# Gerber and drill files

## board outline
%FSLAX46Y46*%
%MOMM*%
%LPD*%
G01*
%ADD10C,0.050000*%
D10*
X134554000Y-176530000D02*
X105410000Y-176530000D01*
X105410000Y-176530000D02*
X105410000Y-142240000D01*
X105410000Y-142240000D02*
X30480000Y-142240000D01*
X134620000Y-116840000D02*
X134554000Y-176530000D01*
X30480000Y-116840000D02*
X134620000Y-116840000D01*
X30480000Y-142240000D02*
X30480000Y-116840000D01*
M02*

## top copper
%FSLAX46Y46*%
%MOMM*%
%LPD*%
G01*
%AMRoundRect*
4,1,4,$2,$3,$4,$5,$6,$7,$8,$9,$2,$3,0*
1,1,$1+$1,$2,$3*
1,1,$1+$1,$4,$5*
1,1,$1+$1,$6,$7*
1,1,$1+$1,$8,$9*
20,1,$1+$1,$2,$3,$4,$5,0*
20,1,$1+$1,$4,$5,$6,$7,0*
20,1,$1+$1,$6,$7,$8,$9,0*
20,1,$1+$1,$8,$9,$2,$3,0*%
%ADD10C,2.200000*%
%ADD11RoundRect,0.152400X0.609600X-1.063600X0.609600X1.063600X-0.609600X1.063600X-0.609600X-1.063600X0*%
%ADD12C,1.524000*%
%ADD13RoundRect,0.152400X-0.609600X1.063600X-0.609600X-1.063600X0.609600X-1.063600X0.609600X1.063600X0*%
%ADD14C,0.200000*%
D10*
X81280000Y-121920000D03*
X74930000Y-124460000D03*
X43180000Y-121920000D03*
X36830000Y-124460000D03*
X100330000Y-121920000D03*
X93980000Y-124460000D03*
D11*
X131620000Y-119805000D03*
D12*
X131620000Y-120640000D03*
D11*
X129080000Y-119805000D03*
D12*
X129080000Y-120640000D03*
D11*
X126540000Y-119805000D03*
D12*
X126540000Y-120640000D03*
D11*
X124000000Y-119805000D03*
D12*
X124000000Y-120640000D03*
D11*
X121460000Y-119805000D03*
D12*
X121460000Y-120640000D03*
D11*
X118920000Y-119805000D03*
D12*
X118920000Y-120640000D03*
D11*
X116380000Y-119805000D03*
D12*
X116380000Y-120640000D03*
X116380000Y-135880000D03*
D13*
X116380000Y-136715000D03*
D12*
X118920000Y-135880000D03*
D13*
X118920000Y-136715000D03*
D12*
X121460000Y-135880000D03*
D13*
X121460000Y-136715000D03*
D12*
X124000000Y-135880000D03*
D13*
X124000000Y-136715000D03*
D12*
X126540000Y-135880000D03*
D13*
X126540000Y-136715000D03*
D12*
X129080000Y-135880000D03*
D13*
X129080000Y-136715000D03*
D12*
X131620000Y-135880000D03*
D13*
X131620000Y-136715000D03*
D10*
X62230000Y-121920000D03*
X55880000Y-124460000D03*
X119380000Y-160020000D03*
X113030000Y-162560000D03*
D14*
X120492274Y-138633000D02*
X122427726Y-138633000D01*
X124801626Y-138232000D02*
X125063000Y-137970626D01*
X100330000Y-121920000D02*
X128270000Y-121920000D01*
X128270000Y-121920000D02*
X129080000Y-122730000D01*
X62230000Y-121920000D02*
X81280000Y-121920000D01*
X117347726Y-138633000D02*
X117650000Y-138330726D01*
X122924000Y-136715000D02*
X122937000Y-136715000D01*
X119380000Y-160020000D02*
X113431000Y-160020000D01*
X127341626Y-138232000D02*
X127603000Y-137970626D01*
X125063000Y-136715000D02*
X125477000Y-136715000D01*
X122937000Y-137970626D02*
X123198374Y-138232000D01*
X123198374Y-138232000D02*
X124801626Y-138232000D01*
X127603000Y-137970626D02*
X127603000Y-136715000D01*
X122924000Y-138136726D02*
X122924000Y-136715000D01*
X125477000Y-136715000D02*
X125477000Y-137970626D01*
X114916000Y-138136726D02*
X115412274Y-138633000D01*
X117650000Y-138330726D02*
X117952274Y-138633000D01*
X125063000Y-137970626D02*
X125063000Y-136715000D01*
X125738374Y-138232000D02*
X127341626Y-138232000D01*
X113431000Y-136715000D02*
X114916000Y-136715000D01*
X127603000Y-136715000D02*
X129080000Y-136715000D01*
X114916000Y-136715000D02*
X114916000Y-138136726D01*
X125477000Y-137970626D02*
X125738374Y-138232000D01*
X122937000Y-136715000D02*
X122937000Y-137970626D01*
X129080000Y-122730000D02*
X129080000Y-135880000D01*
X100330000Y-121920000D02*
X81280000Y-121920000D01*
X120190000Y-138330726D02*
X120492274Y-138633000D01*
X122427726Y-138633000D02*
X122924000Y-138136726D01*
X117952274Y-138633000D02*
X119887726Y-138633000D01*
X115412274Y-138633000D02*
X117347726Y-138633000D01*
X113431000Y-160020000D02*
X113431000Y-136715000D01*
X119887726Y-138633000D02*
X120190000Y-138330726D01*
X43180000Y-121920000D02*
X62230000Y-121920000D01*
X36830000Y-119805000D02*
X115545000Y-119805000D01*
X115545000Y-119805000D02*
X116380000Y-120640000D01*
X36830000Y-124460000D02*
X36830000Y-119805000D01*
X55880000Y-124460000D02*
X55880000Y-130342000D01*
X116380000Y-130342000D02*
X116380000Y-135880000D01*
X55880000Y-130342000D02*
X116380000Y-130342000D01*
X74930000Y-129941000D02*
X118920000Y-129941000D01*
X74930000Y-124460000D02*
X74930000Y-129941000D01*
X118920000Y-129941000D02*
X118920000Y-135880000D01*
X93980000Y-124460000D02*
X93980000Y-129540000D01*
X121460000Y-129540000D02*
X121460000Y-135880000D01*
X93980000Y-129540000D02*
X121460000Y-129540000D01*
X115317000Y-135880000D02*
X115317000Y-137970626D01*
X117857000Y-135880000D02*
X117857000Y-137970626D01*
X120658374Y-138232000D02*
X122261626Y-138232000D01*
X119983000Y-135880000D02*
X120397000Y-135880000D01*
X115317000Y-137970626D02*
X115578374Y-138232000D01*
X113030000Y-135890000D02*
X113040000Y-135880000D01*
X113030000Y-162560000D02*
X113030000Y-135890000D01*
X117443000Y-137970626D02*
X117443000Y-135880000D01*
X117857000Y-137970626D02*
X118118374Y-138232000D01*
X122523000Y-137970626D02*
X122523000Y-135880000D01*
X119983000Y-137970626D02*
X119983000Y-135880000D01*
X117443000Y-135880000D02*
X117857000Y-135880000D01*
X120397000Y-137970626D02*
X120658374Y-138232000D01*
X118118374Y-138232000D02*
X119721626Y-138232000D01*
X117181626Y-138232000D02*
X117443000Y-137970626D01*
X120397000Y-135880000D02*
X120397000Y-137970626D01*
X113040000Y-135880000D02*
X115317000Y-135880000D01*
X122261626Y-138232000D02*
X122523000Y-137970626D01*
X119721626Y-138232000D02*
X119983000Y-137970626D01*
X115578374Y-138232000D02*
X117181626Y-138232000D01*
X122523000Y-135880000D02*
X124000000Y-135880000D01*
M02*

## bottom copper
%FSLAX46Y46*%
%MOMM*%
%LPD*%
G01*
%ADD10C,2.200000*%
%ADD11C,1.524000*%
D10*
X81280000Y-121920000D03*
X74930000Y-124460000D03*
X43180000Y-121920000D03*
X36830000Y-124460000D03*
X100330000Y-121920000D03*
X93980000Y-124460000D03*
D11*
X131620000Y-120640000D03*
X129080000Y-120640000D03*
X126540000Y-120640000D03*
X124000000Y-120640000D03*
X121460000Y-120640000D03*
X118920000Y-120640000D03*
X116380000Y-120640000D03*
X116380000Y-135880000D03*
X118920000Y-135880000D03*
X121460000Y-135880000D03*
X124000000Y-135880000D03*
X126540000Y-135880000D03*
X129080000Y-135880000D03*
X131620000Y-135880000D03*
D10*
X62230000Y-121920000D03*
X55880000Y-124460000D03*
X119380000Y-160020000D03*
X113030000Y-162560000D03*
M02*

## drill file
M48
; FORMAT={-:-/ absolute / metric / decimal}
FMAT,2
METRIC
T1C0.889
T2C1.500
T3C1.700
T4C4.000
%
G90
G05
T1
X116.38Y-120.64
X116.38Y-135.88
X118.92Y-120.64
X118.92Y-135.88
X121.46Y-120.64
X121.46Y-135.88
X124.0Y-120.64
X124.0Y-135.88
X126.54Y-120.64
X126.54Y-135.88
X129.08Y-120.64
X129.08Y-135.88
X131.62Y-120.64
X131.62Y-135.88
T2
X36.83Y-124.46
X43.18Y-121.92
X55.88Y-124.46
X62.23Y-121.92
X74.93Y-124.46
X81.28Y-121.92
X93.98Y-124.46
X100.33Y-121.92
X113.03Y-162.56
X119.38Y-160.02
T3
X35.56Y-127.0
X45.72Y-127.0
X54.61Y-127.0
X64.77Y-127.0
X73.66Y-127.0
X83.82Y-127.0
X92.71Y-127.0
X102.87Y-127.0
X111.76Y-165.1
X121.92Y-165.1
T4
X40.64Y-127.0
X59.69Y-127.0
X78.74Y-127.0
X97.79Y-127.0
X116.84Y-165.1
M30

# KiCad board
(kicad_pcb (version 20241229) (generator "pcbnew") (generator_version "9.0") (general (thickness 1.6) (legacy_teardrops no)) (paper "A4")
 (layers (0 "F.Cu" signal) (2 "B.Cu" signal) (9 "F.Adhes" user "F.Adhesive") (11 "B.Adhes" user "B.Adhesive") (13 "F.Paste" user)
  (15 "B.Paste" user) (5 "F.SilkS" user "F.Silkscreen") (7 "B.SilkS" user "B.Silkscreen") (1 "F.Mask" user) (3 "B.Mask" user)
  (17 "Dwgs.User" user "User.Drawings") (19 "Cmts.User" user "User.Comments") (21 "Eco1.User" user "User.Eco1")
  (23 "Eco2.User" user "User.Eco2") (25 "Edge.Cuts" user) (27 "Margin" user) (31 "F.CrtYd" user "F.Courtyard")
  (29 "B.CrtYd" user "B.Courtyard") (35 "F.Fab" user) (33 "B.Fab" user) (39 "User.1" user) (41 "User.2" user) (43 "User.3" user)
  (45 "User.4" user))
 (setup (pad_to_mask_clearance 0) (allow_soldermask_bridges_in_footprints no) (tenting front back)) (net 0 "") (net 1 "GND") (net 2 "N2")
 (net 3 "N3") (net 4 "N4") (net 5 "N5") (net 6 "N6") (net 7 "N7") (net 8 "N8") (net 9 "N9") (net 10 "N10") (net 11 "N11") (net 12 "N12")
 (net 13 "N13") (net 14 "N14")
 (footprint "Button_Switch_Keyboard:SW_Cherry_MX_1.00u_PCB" (layer "F.Cu") (at 81.28 121.92)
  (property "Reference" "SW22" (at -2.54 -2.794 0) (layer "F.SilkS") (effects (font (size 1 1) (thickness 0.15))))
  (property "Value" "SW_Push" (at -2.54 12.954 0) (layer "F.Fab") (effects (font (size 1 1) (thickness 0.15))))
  (pad "" np_thru_hole circle (at -7.62 5.08) (size 1.7 1.7) (drill 1.7) (layers "*.Cu" "*.Mask"))
  (pad "" np_thru_hole circle (at -2.54 5.08) (size 4 4) (drill 4) (layers "*.Cu" "*.Mask"))
  (pad "" np_thru_hole circle (at 2.54 5.08) (size 1.7 1.7) (drill 1.7) (layers "*.Cu" "*.Mask"))
  (pad "1" thru_hole circle (at 0 0) (size 2.2 2.2) (drill 1.5) (layers "*.Cu" "*.Mask") (remove_unused_layers no) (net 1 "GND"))
  (pad "2" thru_hole circle (at -6.35 2.54) (size 2.2 2.2) (drill 1.5) (layers "*.Cu" "*.Mask") (remove_unused_layers no) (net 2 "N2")))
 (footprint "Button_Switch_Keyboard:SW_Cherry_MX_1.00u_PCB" (layer "F.Cu") (at 43.18 121.92)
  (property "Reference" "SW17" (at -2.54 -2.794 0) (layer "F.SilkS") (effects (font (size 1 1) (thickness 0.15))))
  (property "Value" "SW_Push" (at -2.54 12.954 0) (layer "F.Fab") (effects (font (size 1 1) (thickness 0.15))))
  (pad "" np_thru_hole circle (at -7.62 5.08) (size 1.7 1.7) (drill 1.7) (layers "*.Cu" "*.Mask"))
  (pad "" np_thru_hole circle (at -2.54 5.08) (size 4 4) (drill 4) (layers "*.Cu" "*.Mask"))
  (pad "" np_thru_hole circle (at 2.54 5.08) (size 1.7 1.7) (drill 1.7) (layers "*.Cu" "*.Mask"))
  (pad "1" thru_hole circle (at 0 0) (size 2.2 2.2) (drill 1.5) (layers "*.Cu" "*.Mask") (remove_unused_layers no) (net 1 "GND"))
  (pad "2" thru_hole circle (at -6.35 2.54) (size 2.2 2.2) (drill 1.5) (layers "*.Cu" "*.Mask") (remove_unused_layers no) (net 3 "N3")))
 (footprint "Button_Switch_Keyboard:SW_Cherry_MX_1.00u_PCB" (layer "F.Cu") (at 100.33 121.92)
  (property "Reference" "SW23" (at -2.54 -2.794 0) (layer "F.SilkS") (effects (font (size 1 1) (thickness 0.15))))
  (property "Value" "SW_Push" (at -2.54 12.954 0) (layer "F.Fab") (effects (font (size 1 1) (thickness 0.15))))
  (pad "" np_thru_hole circle (at -7.62 5.08) (size 1.7 1.7) (drill 1.7) (layers "*.Cu" "*.Mask"))
  (pad "" np_thru_hole circle (at -2.54 5.08) (size 4 4) (drill 4) (layers "*.Cu" "*.Mask"))
  (pad "" np_thru_hole circle (at 2.54 5.08) (size 1.7 1.7) (drill 1.7) (layers "*.Cu" "*.Mask"))
  (pad "1" thru_hole circle (at 0 0) (size 2.2 2.2) (drill 1.5) (layers "*.Cu" "*.Mask") (remove_unused_layers no) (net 1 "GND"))
  (pad "2" thru_hole circle (at -6.35 2.54) (size 2.2 2.2) (drill 1.5) (layers "*.Cu" "*.Mask") (remove_unused_layers no) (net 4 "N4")))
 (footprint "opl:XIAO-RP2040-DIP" (layer "F.Cu") (at 124 128.26 -90)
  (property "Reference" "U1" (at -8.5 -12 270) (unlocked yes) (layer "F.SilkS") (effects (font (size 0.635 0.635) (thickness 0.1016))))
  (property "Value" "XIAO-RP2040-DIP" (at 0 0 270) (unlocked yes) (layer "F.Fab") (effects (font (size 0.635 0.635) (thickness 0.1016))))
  (pad "1" smd roundrect (at -8.455 -7.62 90) (size 2.432 1.524) (layers "F.Cu" "F.Mask") (roundrect_rratio 0.1) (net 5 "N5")
   (thermal_bridge_angle 45))
  (pad "1" thru_hole circle (at -7.62 -7.62 90) (size 1.524 1.524) (drill 0.889) (layers "*.Cu" "*.Mask") (remove_unused_layers no)
   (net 5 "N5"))
  (pad "2" smd roundrect (at -8.455 -5.08 90) (size 2.432 1.524) (layers "F.Cu" "F.Mask") (roundrect_rratio 0.1) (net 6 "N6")
   (thermal_bridge_angle 45))
  (pad "2" thru_hole circle (at -7.62 -5.08 90) (size 1.524 1.524) (drill 0.889) (layers "*.Cu" "*.Mask") (remove_unused_layers no)
   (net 6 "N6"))
  (pad "3" smd roundrect (at -8.455 -2.54 90) (size 2.432 1.524) (layers "F.Cu" "F.Mask") (roundrect_rratio 0.1) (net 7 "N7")
   (thermal_bridge_angle 45))
  (pad "3" thru_hole circle (at -7.62 -2.54 90) (size 1.524 1.524) (drill 0.889) (layers "*.Cu" "*.Mask") (remove_unused_layers no)
   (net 7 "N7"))
  (pad "4" smd roundrect (at -8.455 0 90) (size 2.432 1.524) (layers "F.Cu" "F.Mask") (roundrect_rratio 0.1) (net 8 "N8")
   (thermal_bridge_angle 45))
  (pad "4" thru_hole circle (at -7.62 0 90) (size 1.524 1.524) (drill 0.889) (layers "*.Cu" "*.Mask") (remove_unused_layers no) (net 8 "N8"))
  (pad "5" smd roundrect (at -8.455 2.54 90) (size 2.432 1.524) (layers "F.Cu" "F.Mask") (roundrect_rratio 0.1) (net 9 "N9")
   (thermal_bridge_angle 45))
  (pad "5" thru_hole circle (at -7.62 2.54 90) (size 1.524 1.524) (drill 0.889) (layers "*.Cu" "*.Mask") (remove_unused_layers no)
   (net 9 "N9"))
  (pad "6" smd roundrect (at -8.455 5.08 90) (size 2.432 1.524) (layers "F.Cu" "F.Mask") (roundrect_rratio 0.1) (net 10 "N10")
   (thermal_bridge_angle 45))
  (pad "6" thru_hole circle (at -7.62 5.08 90) (size 1.524 1.524) (drill 0.889) (layers "*.Cu" "*.Mask") (remove_unused_layers no)
   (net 10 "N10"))
  (pad "7" smd roundrect (at -8.455 7.62 90) (size 2.432 1.524) (layers "F.Cu" "F.Mask") (roundrect_rratio 0.1) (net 3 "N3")
   (thermal_bridge_angle 45))
  (pad "7" thru_hole circle (at -7.62 7.62 90) (size 1.524 1.524) (drill 0.889) (layers "*.Cu" "*.Mask") (remove_unused_layers no)
   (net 3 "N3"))
  (pad "8" thru_hole circle (at 7.62 7.62 270) (size 1.524 1.524) (drill 0.889) (layers "*.Cu" "*.Mask") (remove_unused_layers no)
   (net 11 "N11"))
  (pad "8" smd roundrect (at 8.455 7.62 270) (size 2.432 1.524) (layers "F.Cu" "F.Mask") (roundrect_rratio 0.1) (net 11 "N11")
   (thermal_bridge_angle 45))
  (pad "9" thru_hole circle (at 7.62 5.08 270) (size 1.524 1.524) (drill 0.889) (layers "*.Cu" "*.Mask") (remove_unused_layers no)
   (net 2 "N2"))
  (pad "9" smd roundrect (at 8.455 5.08 270) (size 2.432 1.524) (layers "F.Cu" "F.Mask") (roundrect_rratio 0.1) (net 2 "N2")
   (thermal_bridge_angle 45))
  (pad "10" thru_hole circle (at 7.62 2.54 270) (size 1.524 1.524) (drill 0.889) (layers "*.Cu" "*.Mask") (remove_unused_layers no)
   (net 4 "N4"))
  (pad "10" smd roundrect (at 8.455 2.54 270) (size 2.432 1.524) (layers "F.Cu" "F.Mask") (roundrect_rratio 0.1) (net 4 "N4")
   (thermal_bridge_angle 45))
  (pad "11" thru_hole circle (at 7.62 0 270) (size 1.524 1.524) (drill 0.889) (layers "*.Cu" "*.Mask") (remove_unused_layers no)
   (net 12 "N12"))
  (pad "11" smd roundrect (at 8.455 0 270) (size 2.432 1.524) (layers "F.Cu" "F.Mask") (roundrect_rratio 0.1) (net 12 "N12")
   (thermal_bridge_angle 45))
  (pad "12" thru_hole circle (at 7.62 -2.54 270) (size 1.524 1.524) (drill 0.889) (layers "*.Cu" "*.Mask") (remove_unused_layers no)
   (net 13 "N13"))
  (pad "12" smd roundrect (at 8.455 -2.54 270) (size 2.432 1.524) (layers "F.Cu" "F.Mask") (roundrect_rratio 0.1) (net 13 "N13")
   (thermal_bridge_angle 45))
  (pad "13" thru_hole circle (at 7.62 -5.08 270) (size 1.524 1.524) (drill 0.889) (layers "*.Cu" "*.Mask") (remove_unused_layers no)
   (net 1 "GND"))
  (pad "13" smd roundrect (at 8.455 -5.08 270) (size 2.432 1.524) (layers "F.Cu" "F.Mask") (roundrect_rratio 0.1) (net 1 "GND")
   (thermal_bridge_angle 45))
  (pad "14" thru_hole circle (at 7.62 -7.62 270) (size 1.524 1.524) (drill 0.889) (layers "*.Cu" "*.Mask") (remove_unused_layers no)
   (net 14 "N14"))
  (pad "14" smd roundrect (at 8.455 -7.62 270) (size 2.432 1.524) (layers "F.Cu" "F.Mask") (roundrect_rratio 0.1) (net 14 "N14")
   (thermal_bridge_angle 45)))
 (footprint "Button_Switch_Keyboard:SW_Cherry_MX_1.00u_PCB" (layer "F.Cu") (at 62.23 121.92)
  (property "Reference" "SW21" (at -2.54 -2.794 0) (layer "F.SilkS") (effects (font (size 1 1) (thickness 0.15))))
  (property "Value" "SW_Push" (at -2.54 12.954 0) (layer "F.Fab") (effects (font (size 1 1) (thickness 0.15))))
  (pad "" np_thru_hole circle (at -7.62 5.08) (size 1.7 1.7) (drill 1.7) (layers "*.Cu" "*.Mask"))
  (pad "" np_thru_hole circle (at -2.54 5.08) (size 4 4) (drill 4) (layers "*.Cu" "*.Mask"))
  (pad "" np_thru_hole circle (at 2.54 5.08) (size 1.7 1.7) (drill 1.7) (layers "*.Cu" "*.Mask"))
  (pad "1" thru_hole circle (at 0 0) (size 2.2 2.2) (drill 1.5) (layers "*.Cu" "*.Mask") (remove_unused_layers no) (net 1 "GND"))
  (pad "2" thru_hole circle (at -6.35 2.54) (size 2.2 2.2) (drill 1.5) (layers "*.Cu" "*.Mask") (remove_unused_layers no) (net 11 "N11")))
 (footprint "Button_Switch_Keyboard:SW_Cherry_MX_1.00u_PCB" (layer "F.Cu") (at 119.38 160.02)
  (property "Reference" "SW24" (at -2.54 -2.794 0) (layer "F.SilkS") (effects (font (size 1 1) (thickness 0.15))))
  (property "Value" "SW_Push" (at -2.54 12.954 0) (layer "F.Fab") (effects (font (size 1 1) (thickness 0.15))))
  (pad "" np_thru_hole circle (at -7.62 5.08) (size 1.7 1.7) (drill 1.7) (layers "*.Cu" "*.Mask"))
  (pad "" np_thru_hole circle (at -2.54 5.08) (size 4 4) (drill 4) (layers "*.Cu" "*.Mask"))
  (pad "" np_thru_hole circle (at 2.54 5.08) (size 1.7 1.7) (drill 1.7) (layers "*.Cu" "*.Mask"))
  (pad "1" thru_hole circle (at 0 0) (size 2.2 2.2) (drill 1.5) (layers "*.Cu" "*.Mask") (remove_unused_layers no) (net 1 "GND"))
  (pad "2" thru_hole circle (at -6.35 2.54) (size 2.2 2.2) (drill 1.5) (layers "*.Cu" "*.Mask") (remove_unused_layers no) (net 12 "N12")))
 (gr_line (start 134.554 176.53) (end 105.41 176.53) (stroke (width 0.05) (type default)) (layer "Edge.Cuts"))
 (gr_line (start 105.41 176.53) (end 105.41 142.24) (stroke (width 0.05) (type default)) (layer "Edge.Cuts"))
 (gr_line (start 105.41 142.24) (end 30.48 142.24) (stroke (width 0.05) (type default)) (layer "Edge.Cuts"))
 (gr_line (start 134.62 116.84) (end 134.554 176.53) (stroke (width 0.05) (type default)) (layer "Edge.Cuts"))
 (gr_line (start 30.48 116.84) (end 134.62 116.84) (stroke (width 0.05) (type default)) (layer "Edge.Cuts"))
 (gr_line (start 30.48 142.24) (end 30.48 116.84) (stroke (width 0.05) (type default)) (layer "Edge.Cuts"))
 (segment (start 120.492274 138.633) (end 122.427726 138.633) (width 0.2) (layer "F.Cu") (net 1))
 (segment (start 124.801626 138.232) (end 125.063 137.970626) (width 0.2) (layer "F.Cu") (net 1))
 (segment (start 100.33 121.92) (end 128.27 121.92) (width 0.2) (layer "F.Cu") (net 1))
 (segment (start 128.27 121.92) (end 129.08 122.73) (width 0.2) (layer "F.Cu") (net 1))
 (segment (start 62.23 121.92) (end 81.28 121.92) (width 0.2) (layer "F.Cu") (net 1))
 (segment (start 117.347726 138.633) (end 117.65 138.330726) (width 0.2) (layer "F.Cu") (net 1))
 (segment (start 122.924 136.715) (end 122.937 136.715) (width 0.2) (layer "F.Cu") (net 1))
 (segment (start 119.38 160.02) (end 113.431 160.02) (width 0.2) (layer "F.Cu") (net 1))
 (segment (start 127.341626 138.232) (end 127.603 137.970626) (width 0.2) (layer "F.Cu") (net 1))
 (segment (start 125.063 136.715) (end 125.477 136.715) (width 0.2) (layer "F.Cu") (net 1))
 (segment (start 122.937 137.970626) (end 123.198374 138.232) (width 0.2) (layer "F.Cu") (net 1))
 (segment (start 123.198374 138.232) (end 124.801626 138.232) (width 0.2) (layer "F.Cu") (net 1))
 (segment (start 127.603 137.970626) (end 127.603 136.715) (width 0.2) (layer "F.Cu") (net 1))
 (segment (start 122.924 138.136726) (end 122.924 136.715) (width 0.2) (layer "F.Cu") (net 1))
 (segment (start 125.477 136.715) (end 125.477 137.970626) (width 0.2) (layer "F.Cu") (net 1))
 (segment (start 114.916 138.136726) (end 115.412274 138.633) (width 0.2) (layer "F.Cu") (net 1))
 (segment (start 117.65 138.330726) (end 117.952274 138.633) (width 0.2) (layer "F.Cu") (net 1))
 (segment (start 125.063 137.970626) (end 125.063 136.715) (width 0.2) (layer "F.Cu") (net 1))
 (segment (start 125.738374 138.232) (end 127.341626 138.232) (width 0.2) (layer "F.Cu") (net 1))
 (segment (start 113.431 136.715) (end 114.916 136.715) (width 0.2) (layer "F.Cu") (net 1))
 (segment (start 127.603 136.715) (end 129.08 136.715) (width 0.2) (layer "F.Cu") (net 1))
 (segment (start 114.916 136.715) (end 114.916 138.136726) (width 0.2) (layer "F.Cu") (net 1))
 (segment (start 125.477 137.970626) (end 125.738374 138.232) (width 0.2) (layer "F.Cu") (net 1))
 (segment (start 122.937 136.715) (end 122.937 137.970626) (width 0.2) (layer "F.Cu") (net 1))
 (segment (start 129.08 122.73) (end 129.08 135.88) (width 0.2) (layer "F.Cu") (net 1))
 (segment (start 100.33 121.92) (end 81.28 121.92) (width 0.2) (layer "F.Cu") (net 1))
 (segment (start 120.19 138.330726) (end 120.492274 138.633) (width 0.2) (layer "F.Cu") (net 1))
 (segment (start 122.427726 138.633) (end 122.924 138.136726) (width 0.2) (layer "F.Cu") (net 1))
 (segment (start 117.952274 138.633) (end 119.887726 138.633) (width 0.2) (layer "F.Cu") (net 1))
 (segment (start 115.412274 138.633) (end 117.347726 138.633) (width 0.2) (layer "F.Cu") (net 1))
 (segment (start 113.431 160.02) (end 113.431 136.715) (width 0.2) (layer "F.Cu") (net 1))
 (segment (start 119.887726 138.633) (end 120.19 138.330726) (width 0.2) (layer "F.Cu") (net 1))
 (segment (start 43.18 121.92) (end 62.23 121.92) (width 0.2) (layer "F.Cu") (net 1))
 (segment (start 36.83 119.805) (end 115.545 119.805) (width 0.2) (layer "F.Cu") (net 3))
 (segment (start 115.545 119.805) (end 116.38 120.64) (width 0.2) (layer "F.Cu") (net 3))
 (segment (start 36.83 124.46) (end 36.83 119.805) (width 0.2) (layer "F.Cu") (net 3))
 (segment (start 55.88 124.46) (end 55.88 130.342) (width 0.2) (layer "F.Cu") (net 11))
 (segment (start 116.38 130.342) (end 116.38 135.88) (width 0.2) (layer "F.Cu") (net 11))
 (segment (start 55.88 130.342) (end 116.38 130.342) (width 0.2) (layer "F.Cu") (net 11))
 (segment (start 74.93 129.941) (end 118.92 129.941) (width 0.2) (layer "F.Cu") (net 2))
 (segment (start 74.93 124.46) (end 74.93 129.941) (width 0.2) (layer "F.Cu") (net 2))
 (segment (start 118.92 129.941) (end 118.92 135.88) (width 0.2) (layer "F.Cu") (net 2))
 (segment (start 93.98 124.46) (end 93.98 129.54) (width 0.2) (layer "F.Cu") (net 4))
 (segment (start 121.46 129.54) (end 121.46 135.88) (width 0.2) (layer "F.Cu") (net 4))
 (segment (start 93.98 129.54) (end 121.46 129.54) (width 0.2) (layer "F.Cu") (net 4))
 (segment (start 115.317 135.88) (end 115.317 137.970626) (width 0.2) (layer "F.Cu") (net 12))
 (segment (start 117.857 135.88) (end 117.857 137.970626) (width 0.2) (layer "F.Cu") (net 12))
 (segment (start 120.658374 138.232) (end 122.261626 138.232) (width 0.2) (layer "F.Cu") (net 12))
 (segment (start 119.983 135.88) (end 120.397 135.88) (width 0.2) (layer "F.Cu") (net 12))
 (segment (start 115.317 137.970626) (end 115.578374 138.232) (width 0.2) (layer "F.Cu") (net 12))
 (segment (start 113.03 135.89) (end 113.04 135.88) (width 0.2) (layer "F.Cu") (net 12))
 (segment (start 113.03 162.56) (end 113.03 135.89) (width 0.2) (layer "F.Cu") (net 12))
 (segment (start 117.443 137.970626) (end 117.443 135.88) (width 0.2) (layer "F.Cu") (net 12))
 (segment (start 117.857 137.970626) (end 118.118374 138.232) (width 0.2) (layer "F.Cu") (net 12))
 (segment (start 122.523 137.970626) (end 122.523 135.88) (width 0.2) (layer "F.Cu") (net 12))
 (segment (start 119.983 137.970626) (end 119.983 135.88) (width 0.2) (layer "F.Cu") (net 12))
 (segment (start 117.443 135.88) (end 117.857 135.88) (width 0.2) (layer "F.Cu") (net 12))
 (segment (start 120.397 137.970626) (end 120.658374 138.232) (width 0.2) (layer "F.Cu") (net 12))
 (segment (start 118.118374 138.232) (end 119.721626 138.232) (width 0.2) (layer "F.Cu") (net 12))
 (segment (start 117.181626 138.232) (end 117.443 137.970626) (width 0.2) (layer "F.Cu") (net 12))
 (segment (start 120.397 135.88) (end 120.397 137.970626) (width 0.2) (layer "F.Cu") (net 12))
 (segment (start 113.04 135.88) (end 115.317 135.88) (width 0.2) (layer "F.Cu") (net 12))
 (segment (start 122.261626 138.232) (end 122.523 137.970626) (width 0.2) (layer "F.Cu") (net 12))
 (segment (start 119.721626 138.232) (end 119.983 137.970626) (width 0.2) (layer "F.Cu") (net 12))
 (segment (start 115.578374 138.232) (end 117.181626 138.232) (width 0.2) (layer "F.Cu") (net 12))
 (segment (start 122.523 135.88) (end 124 135.88) (width 0.2) (layer "F.Cu") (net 12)))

